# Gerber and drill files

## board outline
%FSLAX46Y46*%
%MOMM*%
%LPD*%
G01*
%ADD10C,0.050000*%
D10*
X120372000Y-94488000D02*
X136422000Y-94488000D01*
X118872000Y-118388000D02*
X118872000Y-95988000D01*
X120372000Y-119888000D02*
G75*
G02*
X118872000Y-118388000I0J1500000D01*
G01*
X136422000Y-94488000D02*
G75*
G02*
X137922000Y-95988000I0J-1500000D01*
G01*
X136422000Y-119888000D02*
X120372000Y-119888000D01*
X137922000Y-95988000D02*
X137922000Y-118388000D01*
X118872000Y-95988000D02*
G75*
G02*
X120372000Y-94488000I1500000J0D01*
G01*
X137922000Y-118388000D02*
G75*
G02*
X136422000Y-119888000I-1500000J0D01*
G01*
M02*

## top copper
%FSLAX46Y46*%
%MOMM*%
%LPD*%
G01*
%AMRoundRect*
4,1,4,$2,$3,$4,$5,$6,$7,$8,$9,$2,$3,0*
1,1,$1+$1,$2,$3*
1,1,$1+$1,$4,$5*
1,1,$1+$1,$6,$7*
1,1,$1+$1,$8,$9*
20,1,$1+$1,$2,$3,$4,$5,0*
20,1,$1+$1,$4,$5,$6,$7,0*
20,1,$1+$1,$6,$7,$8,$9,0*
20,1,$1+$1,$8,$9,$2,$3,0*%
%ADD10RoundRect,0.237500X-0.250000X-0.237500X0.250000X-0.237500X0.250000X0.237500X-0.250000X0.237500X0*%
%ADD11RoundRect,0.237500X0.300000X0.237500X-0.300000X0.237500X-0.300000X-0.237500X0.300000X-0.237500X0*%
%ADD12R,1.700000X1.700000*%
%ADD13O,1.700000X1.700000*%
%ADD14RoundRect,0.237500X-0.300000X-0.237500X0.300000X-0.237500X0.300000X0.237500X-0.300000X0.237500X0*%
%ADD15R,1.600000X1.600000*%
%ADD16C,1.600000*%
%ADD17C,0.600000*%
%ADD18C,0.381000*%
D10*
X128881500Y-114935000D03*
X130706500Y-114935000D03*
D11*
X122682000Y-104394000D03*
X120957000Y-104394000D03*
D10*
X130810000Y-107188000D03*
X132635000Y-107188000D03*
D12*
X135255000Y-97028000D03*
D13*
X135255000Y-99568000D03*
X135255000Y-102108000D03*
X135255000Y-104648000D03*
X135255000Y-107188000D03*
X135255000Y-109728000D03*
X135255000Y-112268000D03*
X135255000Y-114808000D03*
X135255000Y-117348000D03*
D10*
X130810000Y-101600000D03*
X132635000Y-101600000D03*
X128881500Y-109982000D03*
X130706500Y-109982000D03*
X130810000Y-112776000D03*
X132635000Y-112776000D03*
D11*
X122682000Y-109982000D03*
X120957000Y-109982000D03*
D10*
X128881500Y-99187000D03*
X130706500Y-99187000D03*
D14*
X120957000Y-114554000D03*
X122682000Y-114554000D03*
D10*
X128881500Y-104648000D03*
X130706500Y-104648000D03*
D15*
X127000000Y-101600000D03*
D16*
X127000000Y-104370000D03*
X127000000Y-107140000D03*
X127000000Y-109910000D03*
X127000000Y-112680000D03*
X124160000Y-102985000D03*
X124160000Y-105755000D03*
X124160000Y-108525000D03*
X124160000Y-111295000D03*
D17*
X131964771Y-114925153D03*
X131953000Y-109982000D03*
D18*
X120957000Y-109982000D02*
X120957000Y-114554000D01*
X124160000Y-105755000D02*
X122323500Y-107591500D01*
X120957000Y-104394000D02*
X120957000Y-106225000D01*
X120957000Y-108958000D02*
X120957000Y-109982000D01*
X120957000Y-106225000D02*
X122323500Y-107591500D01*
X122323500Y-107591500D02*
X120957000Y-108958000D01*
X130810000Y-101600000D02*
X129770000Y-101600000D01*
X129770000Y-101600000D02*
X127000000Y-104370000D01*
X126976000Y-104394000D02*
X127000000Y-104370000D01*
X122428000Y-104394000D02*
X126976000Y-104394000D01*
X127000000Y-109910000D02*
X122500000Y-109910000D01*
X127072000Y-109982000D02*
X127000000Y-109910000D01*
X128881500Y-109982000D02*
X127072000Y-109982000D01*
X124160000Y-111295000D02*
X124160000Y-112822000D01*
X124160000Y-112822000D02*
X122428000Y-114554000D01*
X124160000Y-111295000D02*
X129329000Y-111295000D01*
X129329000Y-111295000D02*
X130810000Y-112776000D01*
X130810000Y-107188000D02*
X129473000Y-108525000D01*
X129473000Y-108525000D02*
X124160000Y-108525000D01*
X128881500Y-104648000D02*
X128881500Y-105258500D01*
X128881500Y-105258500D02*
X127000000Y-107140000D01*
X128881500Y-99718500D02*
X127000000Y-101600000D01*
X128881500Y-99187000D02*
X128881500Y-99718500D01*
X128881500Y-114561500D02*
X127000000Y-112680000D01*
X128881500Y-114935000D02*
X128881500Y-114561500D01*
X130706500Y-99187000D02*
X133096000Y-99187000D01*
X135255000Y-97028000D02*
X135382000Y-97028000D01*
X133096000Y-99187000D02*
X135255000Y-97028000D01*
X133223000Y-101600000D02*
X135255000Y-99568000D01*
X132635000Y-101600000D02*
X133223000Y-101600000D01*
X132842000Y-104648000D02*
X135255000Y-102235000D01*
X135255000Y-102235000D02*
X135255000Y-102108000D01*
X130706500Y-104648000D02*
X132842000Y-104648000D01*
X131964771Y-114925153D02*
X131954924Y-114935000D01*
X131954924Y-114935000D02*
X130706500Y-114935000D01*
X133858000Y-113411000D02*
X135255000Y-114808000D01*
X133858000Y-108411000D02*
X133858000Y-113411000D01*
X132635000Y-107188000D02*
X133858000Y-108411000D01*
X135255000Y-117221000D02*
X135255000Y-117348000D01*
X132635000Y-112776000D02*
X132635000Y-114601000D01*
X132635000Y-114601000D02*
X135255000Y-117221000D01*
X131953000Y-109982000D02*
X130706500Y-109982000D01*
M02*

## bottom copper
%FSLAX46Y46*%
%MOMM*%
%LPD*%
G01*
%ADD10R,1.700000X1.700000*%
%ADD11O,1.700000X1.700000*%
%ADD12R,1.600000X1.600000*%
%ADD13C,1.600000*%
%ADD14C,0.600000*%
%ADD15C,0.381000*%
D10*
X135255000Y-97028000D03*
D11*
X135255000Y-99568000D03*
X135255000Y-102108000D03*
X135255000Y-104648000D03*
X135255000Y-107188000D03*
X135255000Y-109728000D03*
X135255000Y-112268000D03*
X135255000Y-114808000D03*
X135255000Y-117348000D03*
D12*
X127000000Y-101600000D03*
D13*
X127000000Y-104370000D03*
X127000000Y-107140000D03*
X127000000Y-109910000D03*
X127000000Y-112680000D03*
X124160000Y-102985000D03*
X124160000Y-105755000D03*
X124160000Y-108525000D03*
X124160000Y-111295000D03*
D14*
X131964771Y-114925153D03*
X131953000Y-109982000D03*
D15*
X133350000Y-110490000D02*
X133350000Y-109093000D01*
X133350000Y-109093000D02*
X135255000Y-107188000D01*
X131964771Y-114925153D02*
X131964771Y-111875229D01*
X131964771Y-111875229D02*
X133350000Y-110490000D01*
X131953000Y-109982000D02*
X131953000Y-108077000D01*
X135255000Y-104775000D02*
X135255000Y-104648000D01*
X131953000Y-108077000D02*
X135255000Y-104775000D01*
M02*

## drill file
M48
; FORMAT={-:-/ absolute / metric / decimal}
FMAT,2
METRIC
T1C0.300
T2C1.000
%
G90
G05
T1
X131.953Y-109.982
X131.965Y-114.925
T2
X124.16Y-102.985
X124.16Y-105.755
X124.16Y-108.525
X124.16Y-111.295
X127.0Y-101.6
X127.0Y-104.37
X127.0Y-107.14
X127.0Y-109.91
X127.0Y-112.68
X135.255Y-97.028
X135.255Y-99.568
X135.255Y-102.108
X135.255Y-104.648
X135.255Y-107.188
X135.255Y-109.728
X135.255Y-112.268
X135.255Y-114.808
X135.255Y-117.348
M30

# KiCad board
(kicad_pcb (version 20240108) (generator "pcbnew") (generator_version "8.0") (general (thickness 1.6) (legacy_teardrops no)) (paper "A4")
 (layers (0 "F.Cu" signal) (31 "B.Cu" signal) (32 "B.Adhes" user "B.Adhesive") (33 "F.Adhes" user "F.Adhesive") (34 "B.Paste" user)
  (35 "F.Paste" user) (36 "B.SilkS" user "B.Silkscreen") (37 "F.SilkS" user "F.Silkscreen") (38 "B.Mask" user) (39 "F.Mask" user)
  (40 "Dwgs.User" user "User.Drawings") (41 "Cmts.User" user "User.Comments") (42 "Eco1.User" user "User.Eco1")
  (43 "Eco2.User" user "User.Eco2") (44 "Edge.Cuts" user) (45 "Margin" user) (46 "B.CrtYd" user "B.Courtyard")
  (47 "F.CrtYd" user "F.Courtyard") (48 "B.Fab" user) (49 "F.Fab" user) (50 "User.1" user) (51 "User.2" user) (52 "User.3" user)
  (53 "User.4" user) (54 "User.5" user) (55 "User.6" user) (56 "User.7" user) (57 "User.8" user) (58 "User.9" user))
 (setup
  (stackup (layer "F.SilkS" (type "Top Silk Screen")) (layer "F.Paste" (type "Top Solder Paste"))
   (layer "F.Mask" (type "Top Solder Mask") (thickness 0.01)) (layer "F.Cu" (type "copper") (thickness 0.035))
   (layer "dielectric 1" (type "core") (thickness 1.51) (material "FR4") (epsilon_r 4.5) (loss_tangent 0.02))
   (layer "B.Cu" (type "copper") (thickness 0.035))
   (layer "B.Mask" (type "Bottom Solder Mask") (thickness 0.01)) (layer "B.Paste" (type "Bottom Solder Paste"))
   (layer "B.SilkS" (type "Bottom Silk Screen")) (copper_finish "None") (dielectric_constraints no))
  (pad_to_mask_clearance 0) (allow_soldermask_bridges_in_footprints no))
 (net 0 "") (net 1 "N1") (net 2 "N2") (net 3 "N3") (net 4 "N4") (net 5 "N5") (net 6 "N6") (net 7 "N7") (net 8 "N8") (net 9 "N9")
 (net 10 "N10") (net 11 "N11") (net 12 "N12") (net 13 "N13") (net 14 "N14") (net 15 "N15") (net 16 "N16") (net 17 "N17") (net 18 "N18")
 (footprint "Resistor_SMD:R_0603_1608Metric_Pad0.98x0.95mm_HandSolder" (layer "F.Cu") (at 129.794 114.935)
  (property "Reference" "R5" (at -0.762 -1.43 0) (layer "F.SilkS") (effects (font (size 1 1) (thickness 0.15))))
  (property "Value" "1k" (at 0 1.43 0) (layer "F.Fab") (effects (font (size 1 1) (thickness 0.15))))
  (pad "1" smd roundrect (at -0.9125 0) (size 0.975 0.95) (layers "F.Cu" "F.Paste" "F.Mask") (roundrect_rratio 0.25) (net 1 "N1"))
  (pad "2" smd roundrect (at 0.9125 0) (size 0.975 0.95) (layers "F.Cu" "F.Paste" "F.Mask") (roundrect_rratio 0.25) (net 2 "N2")))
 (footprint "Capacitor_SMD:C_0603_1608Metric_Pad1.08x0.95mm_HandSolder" (layer "F.Cu") (at 121.8195 104.394 180)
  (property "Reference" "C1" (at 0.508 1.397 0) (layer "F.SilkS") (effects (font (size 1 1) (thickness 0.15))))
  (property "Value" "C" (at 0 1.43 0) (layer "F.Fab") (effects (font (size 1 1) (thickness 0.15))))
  (pad "1" smd roundrect (at -0.8625 0 180) (size 1.075 0.95) (layers "F.Cu" "F.Paste" "F.Mask") (roundrect_rratio 0.25) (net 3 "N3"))
  (pad "2" smd roundrect (at 0.8625 0 180) (size 1.075 0.95) (layers "F.Cu" "F.Paste" "F.Mask") (roundrect_rratio 0.25) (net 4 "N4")))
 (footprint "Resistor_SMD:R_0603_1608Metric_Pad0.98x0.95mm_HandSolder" (layer "F.Cu") (at 131.7225 107.188)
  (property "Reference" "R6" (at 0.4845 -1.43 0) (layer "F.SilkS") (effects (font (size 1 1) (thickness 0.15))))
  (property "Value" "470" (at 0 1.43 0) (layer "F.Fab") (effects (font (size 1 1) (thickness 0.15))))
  (pad "1" smd roundrect (at -0.9125 0) (size 0.975 0.95) (layers "F.Cu" "F.Paste" "F.Mask") (roundrect_rratio 0.25) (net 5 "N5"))
  (pad "2" smd roundrect (at 0.9125 0) (size 0.975 0.95) (layers "F.Cu" "F.Paste" "F.Mask") (roundrect_rratio 0.25) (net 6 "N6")))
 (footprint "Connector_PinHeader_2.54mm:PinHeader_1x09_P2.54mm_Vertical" (layer "F.Cu") (at 135.255 97.028)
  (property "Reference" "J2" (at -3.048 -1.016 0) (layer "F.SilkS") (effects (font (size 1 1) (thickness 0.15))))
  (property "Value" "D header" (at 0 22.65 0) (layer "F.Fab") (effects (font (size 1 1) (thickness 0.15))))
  (pad "1" thru_hole rect (at 0 0) (size 1.7 1.7) (drill 1) (layers "*.Cu" "*.Mask") (remove_unused_layers no) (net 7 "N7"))
  (pad "2" thru_hole oval (at 0 2.54) (size 1.7 1.7) (drill 1) (layers "*.Cu" "*.Mask") (remove_unused_layers no) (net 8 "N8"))
  (pad "3" thru_hole oval (at 0 5.08) (size 1.7 1.7) (drill 1) (layers "*.Cu" "*.Mask") (remove_unused_layers no) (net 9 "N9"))
  (pad "4" thru_hole oval (at 0 7.62) (size 1.7 1.7) (drill 1) (layers "*.Cu" "*.Mask") (remove_unused_layers no) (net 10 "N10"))
  (pad "5" thru_hole oval (at 0 10.16) (size 1.7 1.7) (drill 1) (layers "*.Cu" "*.Mask") (remove_unused_layers no) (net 2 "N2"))
  (pad "6" thru_hole oval (at 0 12.7) (size 1.7 1.7) (drill 1) (layers "*.Cu" "*.Mask") (remove_unused_layers no) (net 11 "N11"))
  (pad "7" thru_hole oval (at 0 15.24) (size 1.7 1.7) (drill 1) (layers "*.Cu" "*.Mask") (remove_unused_layers no) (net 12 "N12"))
  (pad "8" thru_hole oval (at 0 17.78) (size 1.7 1.7) (drill 1) (layers "*.Cu" "*.Mask") (remove_unused_layers no) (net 6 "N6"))
  (pad "9" thru_hole oval (at 0 20.32) (size 1.7 1.7) (drill 1) (layers "*.Cu" "*.Mask") (remove_unused_layers no) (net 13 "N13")))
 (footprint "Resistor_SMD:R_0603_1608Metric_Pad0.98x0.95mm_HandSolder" (layer "F.Cu") (at 131.7225 101.6)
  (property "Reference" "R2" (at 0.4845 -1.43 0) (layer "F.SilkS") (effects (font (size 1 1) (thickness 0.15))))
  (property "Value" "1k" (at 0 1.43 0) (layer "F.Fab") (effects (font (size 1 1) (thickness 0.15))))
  (pad "1" smd roundrect (at -0.9125 0) (size 0.975 0.95) (layers "F.Cu" "F.Paste" "F.Mask") (roundrect_rratio 0.25) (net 3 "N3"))
  (pad "2" smd roundrect (at 0.9125 0) (size 0.975 0.95) (layers "F.Cu" "F.Paste" "F.Mask") (roundrect_rratio 0.25) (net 8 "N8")))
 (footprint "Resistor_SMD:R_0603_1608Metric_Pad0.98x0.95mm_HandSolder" (layer "F.Cu") (at 129.794 109.982)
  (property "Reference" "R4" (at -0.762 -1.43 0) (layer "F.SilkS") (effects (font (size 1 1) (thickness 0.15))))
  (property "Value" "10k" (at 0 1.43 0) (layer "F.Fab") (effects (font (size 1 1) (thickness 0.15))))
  (pad "1" smd roundrect (at -0.9125 0) (size 0.975 0.95) (layers "F.Cu" "F.Paste" "F.Mask") (roundrect_rratio 0.25) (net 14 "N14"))
  (pad "2" smd roundrect (at 0.9125 0) (size 0.975 0.95) (layers "F.Cu" "F.Paste" "F.Mask") (roundrect_rratio 0.25) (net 10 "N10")))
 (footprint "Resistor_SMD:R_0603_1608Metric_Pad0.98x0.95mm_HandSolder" (layer "F.Cu") (at 131.7225 112.776)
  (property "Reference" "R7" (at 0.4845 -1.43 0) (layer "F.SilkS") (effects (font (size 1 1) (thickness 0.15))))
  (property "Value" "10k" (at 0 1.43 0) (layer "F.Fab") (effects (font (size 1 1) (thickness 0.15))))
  (pad "1" smd roundrect (at -0.9125 0) (size 0.975 0.95) (layers "F.Cu" "F.Paste" "F.Mask") (roundrect_rratio 0.25) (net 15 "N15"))
  (pad "2" smd roundrect (at 0.9125 0) (size 0.975 0.95) (layers "F.Cu" "F.Paste" "F.Mask") (roundrect_rratio 0.25) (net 13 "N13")))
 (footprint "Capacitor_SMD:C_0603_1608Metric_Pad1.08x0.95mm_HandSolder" (layer "F.Cu") (at 121.8195 109.982 180)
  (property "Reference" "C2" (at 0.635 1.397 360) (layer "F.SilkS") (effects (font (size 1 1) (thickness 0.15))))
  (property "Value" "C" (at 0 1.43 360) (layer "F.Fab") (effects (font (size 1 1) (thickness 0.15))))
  (pad "1" smd roundrect (at -0.8625 0 180) (size 1.075 0.95) (layers "F.Cu" "F.Paste" "F.Mask") (roundrect_rratio 0.25) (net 14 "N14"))
  (pad "2" smd roundrect (at 0.8625 0 180) (size 1.075 0.95) (layers "F.Cu" "F.Paste" "F.Mask") (roundrect_rratio 0.25) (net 4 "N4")))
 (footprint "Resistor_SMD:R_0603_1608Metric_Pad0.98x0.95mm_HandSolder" (layer "F.Cu") (at 129.794 99.187)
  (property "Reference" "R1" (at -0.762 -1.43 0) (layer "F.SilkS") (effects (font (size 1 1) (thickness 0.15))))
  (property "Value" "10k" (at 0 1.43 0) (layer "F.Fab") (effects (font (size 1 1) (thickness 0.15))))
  (pad "1" smd roundrect (at -0.9125 0) (size 0.975 0.95) (layers "F.Cu" "F.Paste" "F.Mask") (roundrect_rratio 0.25) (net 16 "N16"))
  (pad "2" smd roundrect (at 0.9125 0) (size 0.975 0.95) (layers "F.Cu" "F.Paste" "F.Mask") (roundrect_rratio 0.25) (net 7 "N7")))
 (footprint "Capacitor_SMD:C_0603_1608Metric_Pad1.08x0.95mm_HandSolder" (layer "F.Cu") (at 121.8195 114.554)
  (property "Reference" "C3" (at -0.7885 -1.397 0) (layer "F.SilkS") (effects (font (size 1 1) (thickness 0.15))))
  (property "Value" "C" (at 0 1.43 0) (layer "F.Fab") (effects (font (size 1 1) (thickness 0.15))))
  (pad "1" smd roundrect (at -0.8625 0) (size 1.075 0.95) (layers "F.Cu" "F.Paste" "F.Mask") (roundrect_rratio 0.25) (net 4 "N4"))
  (pad "2" smd roundrect (at 0.8625 0) (size 1.075 0.95) (layers "F.Cu" "F.Paste" "F.Mask") (roundrect_rratio 0.25) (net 15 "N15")))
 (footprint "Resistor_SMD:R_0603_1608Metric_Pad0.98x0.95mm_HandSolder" (layer "F.Cu") (at 129.794 104.648)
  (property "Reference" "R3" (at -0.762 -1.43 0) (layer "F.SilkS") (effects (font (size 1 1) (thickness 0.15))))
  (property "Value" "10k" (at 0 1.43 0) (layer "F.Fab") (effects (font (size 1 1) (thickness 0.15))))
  (pad "1" smd roundrect (at -0.9125 0) (size 0.975 0.95) (layers "F.Cu" "F.Paste" "F.Mask") (roundrect_rratio 0.25) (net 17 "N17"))
  (pad "2" smd roundrect (at 0.9125 0) (size 0.975 0.95) (layers "F.Cu" "F.Paste" "F.Mask") (roundrect_rratio 0.25) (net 9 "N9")))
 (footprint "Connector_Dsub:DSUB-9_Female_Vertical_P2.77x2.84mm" (layer "B.Cu") (at 127 101.6 90)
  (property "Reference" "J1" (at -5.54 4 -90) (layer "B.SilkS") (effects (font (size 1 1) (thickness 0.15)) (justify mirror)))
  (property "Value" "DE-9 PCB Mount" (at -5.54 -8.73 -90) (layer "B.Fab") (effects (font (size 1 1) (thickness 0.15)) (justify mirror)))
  (pad "1" thru_hole rect (at 0 0 90) (size 1.6 1.6) (drill 1) (layers "*.Cu" "*.Mask") (remove_unused_layers no) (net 16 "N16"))
  (pad "2" thru_hole circle (at -2.77 0 90) (size 1.6 1.6) (drill 1) (layers "*.Cu" "*.Mask") (remove_unused_layers no) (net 3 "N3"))
  (pad "3" thru_hole circle (at -5.54 0 90) (size 1.6 1.6) (drill 1) (layers "*.Cu" "*.Mask") (remove_unused_layers no) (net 17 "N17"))
  (pad "4" thru_hole circle (at -8.31 0 90) (size 1.6 1.6) (drill 1) (layers "*.Cu" "*.Mask") (remove_unused_layers no) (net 14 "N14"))
  (pad "5" thru_hole circle (at -11.08 0 90) (size 1.6 1.6) (drill 1) (layers "*.Cu" "*.Mask") (remove_unused_layers no) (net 1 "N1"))
  (pad "6" thru_hole circle (at -1.385 -2.84 90) (size 1.6 1.6) (drill 1) (layers "*.Cu" "*.Mask") (remove_unused_layers no) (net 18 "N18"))
  (pad "7" thru_hole circle (at -4.155 -2.84 90) (size 1.6 1.6) (drill 1) (layers "*.Cu" "*.Mask") (remove_unused_layers no) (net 4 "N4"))
  (pad "8" thru_hole circle (at -6.925 -2.84 90) (size 1.6 1.6) (drill 1) (layers "*.Cu" "*.Mask") (remove_unused_layers no) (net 5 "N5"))
  (pad "9" thru_hole circle (at -9.695 -2.84 90) (size 1.6 1.6) (drill 1) (layers "*.Cu" "*.Mask") (remove_unused_layers no) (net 15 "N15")))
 (gr_line (start 120.372 94.488) (end 136.422 94.488) (stroke (width 0.05) (type default)) (layer "Edge.Cuts"))
 (gr_line (start 118.872 118.388) (end 118.872 95.988) (stroke (width 0.05) (type default)) (layer "Edge.Cuts"))
 (gr_arc (start 120.372 119.888) (mid 119.31134 119.44866) (end 118.872 118.388) (stroke (width 0.05) (type default)) (layer "Edge.Cuts"))
 (gr_arc (start 136.422 94.488) (mid 137.48266 94.92734) (end 137.922 95.988) (stroke (width 0.05) (type default)) (layer "Edge.Cuts"))
 (gr_line (start 136.422 119.888) (end 120.372 119.888) (stroke (width 0.05) (type default)) (layer "Edge.Cuts"))
 (gr_line (start 137.922 95.988) (end 137.922 118.388) (stroke (width 0.05) (type default)) (layer "Edge.Cuts"))
 (gr_arc (start 118.872 95.988) (mid 119.31134 94.92734) (end 120.372 94.488) (stroke (width 0.05) (type default)) (layer "Edge.Cuts"))
 (gr_arc (start 137.922 118.388) (mid 137.48266 119.44866) (end 136.422 119.888) (stroke (width 0.05) (type default)) (layer "Edge.Cuts"))
 (segment (start 120.957 109.982) (end 120.957 114.554) (width 0.381) (layer "F.Cu") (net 4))
 (segment (start 124.16 105.755) (end 122.3235 107.5915) (width 0.381) (layer "F.Cu") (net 4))
 (segment (start 120.957 104.394) (end 120.957 106.225) (width 0.381) (layer "F.Cu") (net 4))
 (segment (start 120.957 108.958) (end 120.957 109.982) (width 0.381) (layer "F.Cu") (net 4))
 (segment (start 120.957 106.225) (end 122.3235 107.5915) (width 0.381) (layer "F.Cu") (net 4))
 (segment (start 122.3235 107.5915) (end 120.957 108.958) (width 0.381) (layer "F.Cu") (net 4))
 (segment (start 130.81 101.6) (end 129.77 101.6) (width 0.381) (layer "F.Cu") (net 3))
 (segment (start 129.77 101.6) (end 127 104.37) (width 0.381) (layer "F.Cu") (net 3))
 (segment (start 126.976 104.394) (end 127 104.37) (width 0.381) (layer "F.Cu") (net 3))
 (segment (start 122.428 104.394) (end 126.976 104.394) (width 0.381) (layer "F.Cu") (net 3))
 (segment (start 127 109.91) (end 122.5 109.91) (width 0.381) (layer "F.Cu") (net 14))
 (segment (start 127.072 109.982) (end 127 109.91) (width 0.381) (layer "F.Cu") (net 14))
 (segment (start 128.8815 109.982) (end 127.072 109.982) (width 0.381) (layer "F.Cu") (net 14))
 (segment (start 124.16 111.295) (end 124.16 112.822) (width 0.381) (layer "F.Cu") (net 15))
 (segment (start 124.16 112.822) (end 122.428 114.554) (width 0.381) (layer "F.Cu") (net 15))
 (segment (start 124.16 111.295) (end 129.329 111.295) (width 0.381) (layer "F.Cu") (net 15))
 (segment (start 129.329 111.295) (end 130.81 112.776) (width 0.381) (layer "F.Cu") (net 15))
 (segment (start 130.81 107.188) (end 129.473 108.525) (width 0.381) (layer "F.Cu") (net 5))
 (segment (start 129.473 108.525) (end 124.16 108.525) (width 0.381) (layer "F.Cu") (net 5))
 (segment (start 128.8815 104.648) (end 128.8815 105.2585) (width 0.381) (layer "F.Cu") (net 17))
 (segment (start 128.8815 105.2585) (end 127 107.14) (width 0.381) (layer "F.Cu") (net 17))
 (segment (start 128.8815 99.7185) (end 127 101.6) (width 0.381) (layer "F.Cu") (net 16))
 (segment (start 128.8815 99.187) (end 128.8815 99.7185) (width 0.381) (layer "F.Cu") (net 16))
 (segment (start 128.8815 114.5615) (end 127 112.68) (width 0.381) (layer "F.Cu") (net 1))
 (segment (start 128.8815 114.935) (end 128.8815 114.5615) (width 0.381) (layer "F.Cu") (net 1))
 (segment (start 130.7065 99.187) (end 133.096 99.187) (width 0.381) (layer "F.Cu") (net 7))
 (segment (start 135.255 97.028) (end 135.382 97.028) (width 0.381) (layer "F.Cu") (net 7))
 (segment (start 133.096 99.187) (end 135.255 97.028) (width 0.381) (layer "F.Cu") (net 7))
 (segment (start 133.223 101.6) (end 135.255 99.568) (width 0.381) (layer "F.Cu") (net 8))
 (segment (start 132.635 101.6) (end 133.223 101.6) (width 0.381) (layer "F.Cu") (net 8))
 (segment (start 132.842 104.648) (end 135.255 102.235) (width 0.381) (layer "F.Cu") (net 9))
 (segment (start 135.255 102.235) (end 135.255 102.108) (width 0.381) (layer "F.Cu") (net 9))
 (segment (start 130.7065 104.648) (end 132.842 104.648) (width 0.381) (layer "F.Cu") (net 9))
 (segment (start 131.964771 114.925153) (end 131.954924 114.935) (width 0.381) (layer "F.Cu") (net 2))
 (segment (start 131.954924 114.935) (end 130.7065 114.935) (width 0.381) (layer "F.Cu") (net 2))
 (via (at 131.964771 114.925153) (size 0.6) (drill 0.3) (layers "F.Cu" "B.Cu") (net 2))
 (segment (start 133.35 110.49) (end 133.35 109.093) (width 0.381) (layer "B.Cu") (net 2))
 (segment (start 133.35 109.093) (end 135.255 107.188) (width 0.381) (layer "B.Cu") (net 2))
 (segment (start 131.964771 114.925153) (end 131.964771 111.875229) (width 0.381) (layer "B.Cu") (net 2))
 (segment (start 131.964771 111.875229) (end 133.35 110.49) (width 0.381) (layer "B.Cu") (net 2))
 (segment (start 133.858 113.411) (end 135.255 114.808) (width 0.381) (layer "F.Cu") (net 6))
 (segment (start 133.858 108.411) (end 133.858 113.411) (width 0.381) (layer "F.Cu") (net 6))
 (segment (start 132.635 107.188) (end 133.858 108.411) (width 0.381) (layer "F.Cu") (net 6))
 (segment (start 135.255 117.221) (end 135.255 117.348) (width 0.381) (layer "F.Cu") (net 13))
 (segment (start 132.635 112.776) (end 132.635 114.601) (width 0.381) (layer "F.Cu") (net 13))
 (segment (start 132.635 114.601) (end 135.255 117.221) (width 0.381) (layer "F.Cu") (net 13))
 (segment (start 131.953 109.982) (end 130.7065 109.982) (width 0.381) (layer "F.Cu") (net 10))
 (via (at 131.953 109.982) (size 0.6) (drill 0.3) (layers "F.Cu" "B.Cu") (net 10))
 (segment (start 131.953 109.982) (end 131.953 108.077) (width 0.381) (layer "B.Cu") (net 10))
 (segment (start 135.255 104.775) (end 135.255 104.648) (width 0.381) (layer "B.Cu") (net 10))
 (segment (start 131.953 108.077) (end 135.255 104.775) (width 0.381) (layer "B.Cu") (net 10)))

